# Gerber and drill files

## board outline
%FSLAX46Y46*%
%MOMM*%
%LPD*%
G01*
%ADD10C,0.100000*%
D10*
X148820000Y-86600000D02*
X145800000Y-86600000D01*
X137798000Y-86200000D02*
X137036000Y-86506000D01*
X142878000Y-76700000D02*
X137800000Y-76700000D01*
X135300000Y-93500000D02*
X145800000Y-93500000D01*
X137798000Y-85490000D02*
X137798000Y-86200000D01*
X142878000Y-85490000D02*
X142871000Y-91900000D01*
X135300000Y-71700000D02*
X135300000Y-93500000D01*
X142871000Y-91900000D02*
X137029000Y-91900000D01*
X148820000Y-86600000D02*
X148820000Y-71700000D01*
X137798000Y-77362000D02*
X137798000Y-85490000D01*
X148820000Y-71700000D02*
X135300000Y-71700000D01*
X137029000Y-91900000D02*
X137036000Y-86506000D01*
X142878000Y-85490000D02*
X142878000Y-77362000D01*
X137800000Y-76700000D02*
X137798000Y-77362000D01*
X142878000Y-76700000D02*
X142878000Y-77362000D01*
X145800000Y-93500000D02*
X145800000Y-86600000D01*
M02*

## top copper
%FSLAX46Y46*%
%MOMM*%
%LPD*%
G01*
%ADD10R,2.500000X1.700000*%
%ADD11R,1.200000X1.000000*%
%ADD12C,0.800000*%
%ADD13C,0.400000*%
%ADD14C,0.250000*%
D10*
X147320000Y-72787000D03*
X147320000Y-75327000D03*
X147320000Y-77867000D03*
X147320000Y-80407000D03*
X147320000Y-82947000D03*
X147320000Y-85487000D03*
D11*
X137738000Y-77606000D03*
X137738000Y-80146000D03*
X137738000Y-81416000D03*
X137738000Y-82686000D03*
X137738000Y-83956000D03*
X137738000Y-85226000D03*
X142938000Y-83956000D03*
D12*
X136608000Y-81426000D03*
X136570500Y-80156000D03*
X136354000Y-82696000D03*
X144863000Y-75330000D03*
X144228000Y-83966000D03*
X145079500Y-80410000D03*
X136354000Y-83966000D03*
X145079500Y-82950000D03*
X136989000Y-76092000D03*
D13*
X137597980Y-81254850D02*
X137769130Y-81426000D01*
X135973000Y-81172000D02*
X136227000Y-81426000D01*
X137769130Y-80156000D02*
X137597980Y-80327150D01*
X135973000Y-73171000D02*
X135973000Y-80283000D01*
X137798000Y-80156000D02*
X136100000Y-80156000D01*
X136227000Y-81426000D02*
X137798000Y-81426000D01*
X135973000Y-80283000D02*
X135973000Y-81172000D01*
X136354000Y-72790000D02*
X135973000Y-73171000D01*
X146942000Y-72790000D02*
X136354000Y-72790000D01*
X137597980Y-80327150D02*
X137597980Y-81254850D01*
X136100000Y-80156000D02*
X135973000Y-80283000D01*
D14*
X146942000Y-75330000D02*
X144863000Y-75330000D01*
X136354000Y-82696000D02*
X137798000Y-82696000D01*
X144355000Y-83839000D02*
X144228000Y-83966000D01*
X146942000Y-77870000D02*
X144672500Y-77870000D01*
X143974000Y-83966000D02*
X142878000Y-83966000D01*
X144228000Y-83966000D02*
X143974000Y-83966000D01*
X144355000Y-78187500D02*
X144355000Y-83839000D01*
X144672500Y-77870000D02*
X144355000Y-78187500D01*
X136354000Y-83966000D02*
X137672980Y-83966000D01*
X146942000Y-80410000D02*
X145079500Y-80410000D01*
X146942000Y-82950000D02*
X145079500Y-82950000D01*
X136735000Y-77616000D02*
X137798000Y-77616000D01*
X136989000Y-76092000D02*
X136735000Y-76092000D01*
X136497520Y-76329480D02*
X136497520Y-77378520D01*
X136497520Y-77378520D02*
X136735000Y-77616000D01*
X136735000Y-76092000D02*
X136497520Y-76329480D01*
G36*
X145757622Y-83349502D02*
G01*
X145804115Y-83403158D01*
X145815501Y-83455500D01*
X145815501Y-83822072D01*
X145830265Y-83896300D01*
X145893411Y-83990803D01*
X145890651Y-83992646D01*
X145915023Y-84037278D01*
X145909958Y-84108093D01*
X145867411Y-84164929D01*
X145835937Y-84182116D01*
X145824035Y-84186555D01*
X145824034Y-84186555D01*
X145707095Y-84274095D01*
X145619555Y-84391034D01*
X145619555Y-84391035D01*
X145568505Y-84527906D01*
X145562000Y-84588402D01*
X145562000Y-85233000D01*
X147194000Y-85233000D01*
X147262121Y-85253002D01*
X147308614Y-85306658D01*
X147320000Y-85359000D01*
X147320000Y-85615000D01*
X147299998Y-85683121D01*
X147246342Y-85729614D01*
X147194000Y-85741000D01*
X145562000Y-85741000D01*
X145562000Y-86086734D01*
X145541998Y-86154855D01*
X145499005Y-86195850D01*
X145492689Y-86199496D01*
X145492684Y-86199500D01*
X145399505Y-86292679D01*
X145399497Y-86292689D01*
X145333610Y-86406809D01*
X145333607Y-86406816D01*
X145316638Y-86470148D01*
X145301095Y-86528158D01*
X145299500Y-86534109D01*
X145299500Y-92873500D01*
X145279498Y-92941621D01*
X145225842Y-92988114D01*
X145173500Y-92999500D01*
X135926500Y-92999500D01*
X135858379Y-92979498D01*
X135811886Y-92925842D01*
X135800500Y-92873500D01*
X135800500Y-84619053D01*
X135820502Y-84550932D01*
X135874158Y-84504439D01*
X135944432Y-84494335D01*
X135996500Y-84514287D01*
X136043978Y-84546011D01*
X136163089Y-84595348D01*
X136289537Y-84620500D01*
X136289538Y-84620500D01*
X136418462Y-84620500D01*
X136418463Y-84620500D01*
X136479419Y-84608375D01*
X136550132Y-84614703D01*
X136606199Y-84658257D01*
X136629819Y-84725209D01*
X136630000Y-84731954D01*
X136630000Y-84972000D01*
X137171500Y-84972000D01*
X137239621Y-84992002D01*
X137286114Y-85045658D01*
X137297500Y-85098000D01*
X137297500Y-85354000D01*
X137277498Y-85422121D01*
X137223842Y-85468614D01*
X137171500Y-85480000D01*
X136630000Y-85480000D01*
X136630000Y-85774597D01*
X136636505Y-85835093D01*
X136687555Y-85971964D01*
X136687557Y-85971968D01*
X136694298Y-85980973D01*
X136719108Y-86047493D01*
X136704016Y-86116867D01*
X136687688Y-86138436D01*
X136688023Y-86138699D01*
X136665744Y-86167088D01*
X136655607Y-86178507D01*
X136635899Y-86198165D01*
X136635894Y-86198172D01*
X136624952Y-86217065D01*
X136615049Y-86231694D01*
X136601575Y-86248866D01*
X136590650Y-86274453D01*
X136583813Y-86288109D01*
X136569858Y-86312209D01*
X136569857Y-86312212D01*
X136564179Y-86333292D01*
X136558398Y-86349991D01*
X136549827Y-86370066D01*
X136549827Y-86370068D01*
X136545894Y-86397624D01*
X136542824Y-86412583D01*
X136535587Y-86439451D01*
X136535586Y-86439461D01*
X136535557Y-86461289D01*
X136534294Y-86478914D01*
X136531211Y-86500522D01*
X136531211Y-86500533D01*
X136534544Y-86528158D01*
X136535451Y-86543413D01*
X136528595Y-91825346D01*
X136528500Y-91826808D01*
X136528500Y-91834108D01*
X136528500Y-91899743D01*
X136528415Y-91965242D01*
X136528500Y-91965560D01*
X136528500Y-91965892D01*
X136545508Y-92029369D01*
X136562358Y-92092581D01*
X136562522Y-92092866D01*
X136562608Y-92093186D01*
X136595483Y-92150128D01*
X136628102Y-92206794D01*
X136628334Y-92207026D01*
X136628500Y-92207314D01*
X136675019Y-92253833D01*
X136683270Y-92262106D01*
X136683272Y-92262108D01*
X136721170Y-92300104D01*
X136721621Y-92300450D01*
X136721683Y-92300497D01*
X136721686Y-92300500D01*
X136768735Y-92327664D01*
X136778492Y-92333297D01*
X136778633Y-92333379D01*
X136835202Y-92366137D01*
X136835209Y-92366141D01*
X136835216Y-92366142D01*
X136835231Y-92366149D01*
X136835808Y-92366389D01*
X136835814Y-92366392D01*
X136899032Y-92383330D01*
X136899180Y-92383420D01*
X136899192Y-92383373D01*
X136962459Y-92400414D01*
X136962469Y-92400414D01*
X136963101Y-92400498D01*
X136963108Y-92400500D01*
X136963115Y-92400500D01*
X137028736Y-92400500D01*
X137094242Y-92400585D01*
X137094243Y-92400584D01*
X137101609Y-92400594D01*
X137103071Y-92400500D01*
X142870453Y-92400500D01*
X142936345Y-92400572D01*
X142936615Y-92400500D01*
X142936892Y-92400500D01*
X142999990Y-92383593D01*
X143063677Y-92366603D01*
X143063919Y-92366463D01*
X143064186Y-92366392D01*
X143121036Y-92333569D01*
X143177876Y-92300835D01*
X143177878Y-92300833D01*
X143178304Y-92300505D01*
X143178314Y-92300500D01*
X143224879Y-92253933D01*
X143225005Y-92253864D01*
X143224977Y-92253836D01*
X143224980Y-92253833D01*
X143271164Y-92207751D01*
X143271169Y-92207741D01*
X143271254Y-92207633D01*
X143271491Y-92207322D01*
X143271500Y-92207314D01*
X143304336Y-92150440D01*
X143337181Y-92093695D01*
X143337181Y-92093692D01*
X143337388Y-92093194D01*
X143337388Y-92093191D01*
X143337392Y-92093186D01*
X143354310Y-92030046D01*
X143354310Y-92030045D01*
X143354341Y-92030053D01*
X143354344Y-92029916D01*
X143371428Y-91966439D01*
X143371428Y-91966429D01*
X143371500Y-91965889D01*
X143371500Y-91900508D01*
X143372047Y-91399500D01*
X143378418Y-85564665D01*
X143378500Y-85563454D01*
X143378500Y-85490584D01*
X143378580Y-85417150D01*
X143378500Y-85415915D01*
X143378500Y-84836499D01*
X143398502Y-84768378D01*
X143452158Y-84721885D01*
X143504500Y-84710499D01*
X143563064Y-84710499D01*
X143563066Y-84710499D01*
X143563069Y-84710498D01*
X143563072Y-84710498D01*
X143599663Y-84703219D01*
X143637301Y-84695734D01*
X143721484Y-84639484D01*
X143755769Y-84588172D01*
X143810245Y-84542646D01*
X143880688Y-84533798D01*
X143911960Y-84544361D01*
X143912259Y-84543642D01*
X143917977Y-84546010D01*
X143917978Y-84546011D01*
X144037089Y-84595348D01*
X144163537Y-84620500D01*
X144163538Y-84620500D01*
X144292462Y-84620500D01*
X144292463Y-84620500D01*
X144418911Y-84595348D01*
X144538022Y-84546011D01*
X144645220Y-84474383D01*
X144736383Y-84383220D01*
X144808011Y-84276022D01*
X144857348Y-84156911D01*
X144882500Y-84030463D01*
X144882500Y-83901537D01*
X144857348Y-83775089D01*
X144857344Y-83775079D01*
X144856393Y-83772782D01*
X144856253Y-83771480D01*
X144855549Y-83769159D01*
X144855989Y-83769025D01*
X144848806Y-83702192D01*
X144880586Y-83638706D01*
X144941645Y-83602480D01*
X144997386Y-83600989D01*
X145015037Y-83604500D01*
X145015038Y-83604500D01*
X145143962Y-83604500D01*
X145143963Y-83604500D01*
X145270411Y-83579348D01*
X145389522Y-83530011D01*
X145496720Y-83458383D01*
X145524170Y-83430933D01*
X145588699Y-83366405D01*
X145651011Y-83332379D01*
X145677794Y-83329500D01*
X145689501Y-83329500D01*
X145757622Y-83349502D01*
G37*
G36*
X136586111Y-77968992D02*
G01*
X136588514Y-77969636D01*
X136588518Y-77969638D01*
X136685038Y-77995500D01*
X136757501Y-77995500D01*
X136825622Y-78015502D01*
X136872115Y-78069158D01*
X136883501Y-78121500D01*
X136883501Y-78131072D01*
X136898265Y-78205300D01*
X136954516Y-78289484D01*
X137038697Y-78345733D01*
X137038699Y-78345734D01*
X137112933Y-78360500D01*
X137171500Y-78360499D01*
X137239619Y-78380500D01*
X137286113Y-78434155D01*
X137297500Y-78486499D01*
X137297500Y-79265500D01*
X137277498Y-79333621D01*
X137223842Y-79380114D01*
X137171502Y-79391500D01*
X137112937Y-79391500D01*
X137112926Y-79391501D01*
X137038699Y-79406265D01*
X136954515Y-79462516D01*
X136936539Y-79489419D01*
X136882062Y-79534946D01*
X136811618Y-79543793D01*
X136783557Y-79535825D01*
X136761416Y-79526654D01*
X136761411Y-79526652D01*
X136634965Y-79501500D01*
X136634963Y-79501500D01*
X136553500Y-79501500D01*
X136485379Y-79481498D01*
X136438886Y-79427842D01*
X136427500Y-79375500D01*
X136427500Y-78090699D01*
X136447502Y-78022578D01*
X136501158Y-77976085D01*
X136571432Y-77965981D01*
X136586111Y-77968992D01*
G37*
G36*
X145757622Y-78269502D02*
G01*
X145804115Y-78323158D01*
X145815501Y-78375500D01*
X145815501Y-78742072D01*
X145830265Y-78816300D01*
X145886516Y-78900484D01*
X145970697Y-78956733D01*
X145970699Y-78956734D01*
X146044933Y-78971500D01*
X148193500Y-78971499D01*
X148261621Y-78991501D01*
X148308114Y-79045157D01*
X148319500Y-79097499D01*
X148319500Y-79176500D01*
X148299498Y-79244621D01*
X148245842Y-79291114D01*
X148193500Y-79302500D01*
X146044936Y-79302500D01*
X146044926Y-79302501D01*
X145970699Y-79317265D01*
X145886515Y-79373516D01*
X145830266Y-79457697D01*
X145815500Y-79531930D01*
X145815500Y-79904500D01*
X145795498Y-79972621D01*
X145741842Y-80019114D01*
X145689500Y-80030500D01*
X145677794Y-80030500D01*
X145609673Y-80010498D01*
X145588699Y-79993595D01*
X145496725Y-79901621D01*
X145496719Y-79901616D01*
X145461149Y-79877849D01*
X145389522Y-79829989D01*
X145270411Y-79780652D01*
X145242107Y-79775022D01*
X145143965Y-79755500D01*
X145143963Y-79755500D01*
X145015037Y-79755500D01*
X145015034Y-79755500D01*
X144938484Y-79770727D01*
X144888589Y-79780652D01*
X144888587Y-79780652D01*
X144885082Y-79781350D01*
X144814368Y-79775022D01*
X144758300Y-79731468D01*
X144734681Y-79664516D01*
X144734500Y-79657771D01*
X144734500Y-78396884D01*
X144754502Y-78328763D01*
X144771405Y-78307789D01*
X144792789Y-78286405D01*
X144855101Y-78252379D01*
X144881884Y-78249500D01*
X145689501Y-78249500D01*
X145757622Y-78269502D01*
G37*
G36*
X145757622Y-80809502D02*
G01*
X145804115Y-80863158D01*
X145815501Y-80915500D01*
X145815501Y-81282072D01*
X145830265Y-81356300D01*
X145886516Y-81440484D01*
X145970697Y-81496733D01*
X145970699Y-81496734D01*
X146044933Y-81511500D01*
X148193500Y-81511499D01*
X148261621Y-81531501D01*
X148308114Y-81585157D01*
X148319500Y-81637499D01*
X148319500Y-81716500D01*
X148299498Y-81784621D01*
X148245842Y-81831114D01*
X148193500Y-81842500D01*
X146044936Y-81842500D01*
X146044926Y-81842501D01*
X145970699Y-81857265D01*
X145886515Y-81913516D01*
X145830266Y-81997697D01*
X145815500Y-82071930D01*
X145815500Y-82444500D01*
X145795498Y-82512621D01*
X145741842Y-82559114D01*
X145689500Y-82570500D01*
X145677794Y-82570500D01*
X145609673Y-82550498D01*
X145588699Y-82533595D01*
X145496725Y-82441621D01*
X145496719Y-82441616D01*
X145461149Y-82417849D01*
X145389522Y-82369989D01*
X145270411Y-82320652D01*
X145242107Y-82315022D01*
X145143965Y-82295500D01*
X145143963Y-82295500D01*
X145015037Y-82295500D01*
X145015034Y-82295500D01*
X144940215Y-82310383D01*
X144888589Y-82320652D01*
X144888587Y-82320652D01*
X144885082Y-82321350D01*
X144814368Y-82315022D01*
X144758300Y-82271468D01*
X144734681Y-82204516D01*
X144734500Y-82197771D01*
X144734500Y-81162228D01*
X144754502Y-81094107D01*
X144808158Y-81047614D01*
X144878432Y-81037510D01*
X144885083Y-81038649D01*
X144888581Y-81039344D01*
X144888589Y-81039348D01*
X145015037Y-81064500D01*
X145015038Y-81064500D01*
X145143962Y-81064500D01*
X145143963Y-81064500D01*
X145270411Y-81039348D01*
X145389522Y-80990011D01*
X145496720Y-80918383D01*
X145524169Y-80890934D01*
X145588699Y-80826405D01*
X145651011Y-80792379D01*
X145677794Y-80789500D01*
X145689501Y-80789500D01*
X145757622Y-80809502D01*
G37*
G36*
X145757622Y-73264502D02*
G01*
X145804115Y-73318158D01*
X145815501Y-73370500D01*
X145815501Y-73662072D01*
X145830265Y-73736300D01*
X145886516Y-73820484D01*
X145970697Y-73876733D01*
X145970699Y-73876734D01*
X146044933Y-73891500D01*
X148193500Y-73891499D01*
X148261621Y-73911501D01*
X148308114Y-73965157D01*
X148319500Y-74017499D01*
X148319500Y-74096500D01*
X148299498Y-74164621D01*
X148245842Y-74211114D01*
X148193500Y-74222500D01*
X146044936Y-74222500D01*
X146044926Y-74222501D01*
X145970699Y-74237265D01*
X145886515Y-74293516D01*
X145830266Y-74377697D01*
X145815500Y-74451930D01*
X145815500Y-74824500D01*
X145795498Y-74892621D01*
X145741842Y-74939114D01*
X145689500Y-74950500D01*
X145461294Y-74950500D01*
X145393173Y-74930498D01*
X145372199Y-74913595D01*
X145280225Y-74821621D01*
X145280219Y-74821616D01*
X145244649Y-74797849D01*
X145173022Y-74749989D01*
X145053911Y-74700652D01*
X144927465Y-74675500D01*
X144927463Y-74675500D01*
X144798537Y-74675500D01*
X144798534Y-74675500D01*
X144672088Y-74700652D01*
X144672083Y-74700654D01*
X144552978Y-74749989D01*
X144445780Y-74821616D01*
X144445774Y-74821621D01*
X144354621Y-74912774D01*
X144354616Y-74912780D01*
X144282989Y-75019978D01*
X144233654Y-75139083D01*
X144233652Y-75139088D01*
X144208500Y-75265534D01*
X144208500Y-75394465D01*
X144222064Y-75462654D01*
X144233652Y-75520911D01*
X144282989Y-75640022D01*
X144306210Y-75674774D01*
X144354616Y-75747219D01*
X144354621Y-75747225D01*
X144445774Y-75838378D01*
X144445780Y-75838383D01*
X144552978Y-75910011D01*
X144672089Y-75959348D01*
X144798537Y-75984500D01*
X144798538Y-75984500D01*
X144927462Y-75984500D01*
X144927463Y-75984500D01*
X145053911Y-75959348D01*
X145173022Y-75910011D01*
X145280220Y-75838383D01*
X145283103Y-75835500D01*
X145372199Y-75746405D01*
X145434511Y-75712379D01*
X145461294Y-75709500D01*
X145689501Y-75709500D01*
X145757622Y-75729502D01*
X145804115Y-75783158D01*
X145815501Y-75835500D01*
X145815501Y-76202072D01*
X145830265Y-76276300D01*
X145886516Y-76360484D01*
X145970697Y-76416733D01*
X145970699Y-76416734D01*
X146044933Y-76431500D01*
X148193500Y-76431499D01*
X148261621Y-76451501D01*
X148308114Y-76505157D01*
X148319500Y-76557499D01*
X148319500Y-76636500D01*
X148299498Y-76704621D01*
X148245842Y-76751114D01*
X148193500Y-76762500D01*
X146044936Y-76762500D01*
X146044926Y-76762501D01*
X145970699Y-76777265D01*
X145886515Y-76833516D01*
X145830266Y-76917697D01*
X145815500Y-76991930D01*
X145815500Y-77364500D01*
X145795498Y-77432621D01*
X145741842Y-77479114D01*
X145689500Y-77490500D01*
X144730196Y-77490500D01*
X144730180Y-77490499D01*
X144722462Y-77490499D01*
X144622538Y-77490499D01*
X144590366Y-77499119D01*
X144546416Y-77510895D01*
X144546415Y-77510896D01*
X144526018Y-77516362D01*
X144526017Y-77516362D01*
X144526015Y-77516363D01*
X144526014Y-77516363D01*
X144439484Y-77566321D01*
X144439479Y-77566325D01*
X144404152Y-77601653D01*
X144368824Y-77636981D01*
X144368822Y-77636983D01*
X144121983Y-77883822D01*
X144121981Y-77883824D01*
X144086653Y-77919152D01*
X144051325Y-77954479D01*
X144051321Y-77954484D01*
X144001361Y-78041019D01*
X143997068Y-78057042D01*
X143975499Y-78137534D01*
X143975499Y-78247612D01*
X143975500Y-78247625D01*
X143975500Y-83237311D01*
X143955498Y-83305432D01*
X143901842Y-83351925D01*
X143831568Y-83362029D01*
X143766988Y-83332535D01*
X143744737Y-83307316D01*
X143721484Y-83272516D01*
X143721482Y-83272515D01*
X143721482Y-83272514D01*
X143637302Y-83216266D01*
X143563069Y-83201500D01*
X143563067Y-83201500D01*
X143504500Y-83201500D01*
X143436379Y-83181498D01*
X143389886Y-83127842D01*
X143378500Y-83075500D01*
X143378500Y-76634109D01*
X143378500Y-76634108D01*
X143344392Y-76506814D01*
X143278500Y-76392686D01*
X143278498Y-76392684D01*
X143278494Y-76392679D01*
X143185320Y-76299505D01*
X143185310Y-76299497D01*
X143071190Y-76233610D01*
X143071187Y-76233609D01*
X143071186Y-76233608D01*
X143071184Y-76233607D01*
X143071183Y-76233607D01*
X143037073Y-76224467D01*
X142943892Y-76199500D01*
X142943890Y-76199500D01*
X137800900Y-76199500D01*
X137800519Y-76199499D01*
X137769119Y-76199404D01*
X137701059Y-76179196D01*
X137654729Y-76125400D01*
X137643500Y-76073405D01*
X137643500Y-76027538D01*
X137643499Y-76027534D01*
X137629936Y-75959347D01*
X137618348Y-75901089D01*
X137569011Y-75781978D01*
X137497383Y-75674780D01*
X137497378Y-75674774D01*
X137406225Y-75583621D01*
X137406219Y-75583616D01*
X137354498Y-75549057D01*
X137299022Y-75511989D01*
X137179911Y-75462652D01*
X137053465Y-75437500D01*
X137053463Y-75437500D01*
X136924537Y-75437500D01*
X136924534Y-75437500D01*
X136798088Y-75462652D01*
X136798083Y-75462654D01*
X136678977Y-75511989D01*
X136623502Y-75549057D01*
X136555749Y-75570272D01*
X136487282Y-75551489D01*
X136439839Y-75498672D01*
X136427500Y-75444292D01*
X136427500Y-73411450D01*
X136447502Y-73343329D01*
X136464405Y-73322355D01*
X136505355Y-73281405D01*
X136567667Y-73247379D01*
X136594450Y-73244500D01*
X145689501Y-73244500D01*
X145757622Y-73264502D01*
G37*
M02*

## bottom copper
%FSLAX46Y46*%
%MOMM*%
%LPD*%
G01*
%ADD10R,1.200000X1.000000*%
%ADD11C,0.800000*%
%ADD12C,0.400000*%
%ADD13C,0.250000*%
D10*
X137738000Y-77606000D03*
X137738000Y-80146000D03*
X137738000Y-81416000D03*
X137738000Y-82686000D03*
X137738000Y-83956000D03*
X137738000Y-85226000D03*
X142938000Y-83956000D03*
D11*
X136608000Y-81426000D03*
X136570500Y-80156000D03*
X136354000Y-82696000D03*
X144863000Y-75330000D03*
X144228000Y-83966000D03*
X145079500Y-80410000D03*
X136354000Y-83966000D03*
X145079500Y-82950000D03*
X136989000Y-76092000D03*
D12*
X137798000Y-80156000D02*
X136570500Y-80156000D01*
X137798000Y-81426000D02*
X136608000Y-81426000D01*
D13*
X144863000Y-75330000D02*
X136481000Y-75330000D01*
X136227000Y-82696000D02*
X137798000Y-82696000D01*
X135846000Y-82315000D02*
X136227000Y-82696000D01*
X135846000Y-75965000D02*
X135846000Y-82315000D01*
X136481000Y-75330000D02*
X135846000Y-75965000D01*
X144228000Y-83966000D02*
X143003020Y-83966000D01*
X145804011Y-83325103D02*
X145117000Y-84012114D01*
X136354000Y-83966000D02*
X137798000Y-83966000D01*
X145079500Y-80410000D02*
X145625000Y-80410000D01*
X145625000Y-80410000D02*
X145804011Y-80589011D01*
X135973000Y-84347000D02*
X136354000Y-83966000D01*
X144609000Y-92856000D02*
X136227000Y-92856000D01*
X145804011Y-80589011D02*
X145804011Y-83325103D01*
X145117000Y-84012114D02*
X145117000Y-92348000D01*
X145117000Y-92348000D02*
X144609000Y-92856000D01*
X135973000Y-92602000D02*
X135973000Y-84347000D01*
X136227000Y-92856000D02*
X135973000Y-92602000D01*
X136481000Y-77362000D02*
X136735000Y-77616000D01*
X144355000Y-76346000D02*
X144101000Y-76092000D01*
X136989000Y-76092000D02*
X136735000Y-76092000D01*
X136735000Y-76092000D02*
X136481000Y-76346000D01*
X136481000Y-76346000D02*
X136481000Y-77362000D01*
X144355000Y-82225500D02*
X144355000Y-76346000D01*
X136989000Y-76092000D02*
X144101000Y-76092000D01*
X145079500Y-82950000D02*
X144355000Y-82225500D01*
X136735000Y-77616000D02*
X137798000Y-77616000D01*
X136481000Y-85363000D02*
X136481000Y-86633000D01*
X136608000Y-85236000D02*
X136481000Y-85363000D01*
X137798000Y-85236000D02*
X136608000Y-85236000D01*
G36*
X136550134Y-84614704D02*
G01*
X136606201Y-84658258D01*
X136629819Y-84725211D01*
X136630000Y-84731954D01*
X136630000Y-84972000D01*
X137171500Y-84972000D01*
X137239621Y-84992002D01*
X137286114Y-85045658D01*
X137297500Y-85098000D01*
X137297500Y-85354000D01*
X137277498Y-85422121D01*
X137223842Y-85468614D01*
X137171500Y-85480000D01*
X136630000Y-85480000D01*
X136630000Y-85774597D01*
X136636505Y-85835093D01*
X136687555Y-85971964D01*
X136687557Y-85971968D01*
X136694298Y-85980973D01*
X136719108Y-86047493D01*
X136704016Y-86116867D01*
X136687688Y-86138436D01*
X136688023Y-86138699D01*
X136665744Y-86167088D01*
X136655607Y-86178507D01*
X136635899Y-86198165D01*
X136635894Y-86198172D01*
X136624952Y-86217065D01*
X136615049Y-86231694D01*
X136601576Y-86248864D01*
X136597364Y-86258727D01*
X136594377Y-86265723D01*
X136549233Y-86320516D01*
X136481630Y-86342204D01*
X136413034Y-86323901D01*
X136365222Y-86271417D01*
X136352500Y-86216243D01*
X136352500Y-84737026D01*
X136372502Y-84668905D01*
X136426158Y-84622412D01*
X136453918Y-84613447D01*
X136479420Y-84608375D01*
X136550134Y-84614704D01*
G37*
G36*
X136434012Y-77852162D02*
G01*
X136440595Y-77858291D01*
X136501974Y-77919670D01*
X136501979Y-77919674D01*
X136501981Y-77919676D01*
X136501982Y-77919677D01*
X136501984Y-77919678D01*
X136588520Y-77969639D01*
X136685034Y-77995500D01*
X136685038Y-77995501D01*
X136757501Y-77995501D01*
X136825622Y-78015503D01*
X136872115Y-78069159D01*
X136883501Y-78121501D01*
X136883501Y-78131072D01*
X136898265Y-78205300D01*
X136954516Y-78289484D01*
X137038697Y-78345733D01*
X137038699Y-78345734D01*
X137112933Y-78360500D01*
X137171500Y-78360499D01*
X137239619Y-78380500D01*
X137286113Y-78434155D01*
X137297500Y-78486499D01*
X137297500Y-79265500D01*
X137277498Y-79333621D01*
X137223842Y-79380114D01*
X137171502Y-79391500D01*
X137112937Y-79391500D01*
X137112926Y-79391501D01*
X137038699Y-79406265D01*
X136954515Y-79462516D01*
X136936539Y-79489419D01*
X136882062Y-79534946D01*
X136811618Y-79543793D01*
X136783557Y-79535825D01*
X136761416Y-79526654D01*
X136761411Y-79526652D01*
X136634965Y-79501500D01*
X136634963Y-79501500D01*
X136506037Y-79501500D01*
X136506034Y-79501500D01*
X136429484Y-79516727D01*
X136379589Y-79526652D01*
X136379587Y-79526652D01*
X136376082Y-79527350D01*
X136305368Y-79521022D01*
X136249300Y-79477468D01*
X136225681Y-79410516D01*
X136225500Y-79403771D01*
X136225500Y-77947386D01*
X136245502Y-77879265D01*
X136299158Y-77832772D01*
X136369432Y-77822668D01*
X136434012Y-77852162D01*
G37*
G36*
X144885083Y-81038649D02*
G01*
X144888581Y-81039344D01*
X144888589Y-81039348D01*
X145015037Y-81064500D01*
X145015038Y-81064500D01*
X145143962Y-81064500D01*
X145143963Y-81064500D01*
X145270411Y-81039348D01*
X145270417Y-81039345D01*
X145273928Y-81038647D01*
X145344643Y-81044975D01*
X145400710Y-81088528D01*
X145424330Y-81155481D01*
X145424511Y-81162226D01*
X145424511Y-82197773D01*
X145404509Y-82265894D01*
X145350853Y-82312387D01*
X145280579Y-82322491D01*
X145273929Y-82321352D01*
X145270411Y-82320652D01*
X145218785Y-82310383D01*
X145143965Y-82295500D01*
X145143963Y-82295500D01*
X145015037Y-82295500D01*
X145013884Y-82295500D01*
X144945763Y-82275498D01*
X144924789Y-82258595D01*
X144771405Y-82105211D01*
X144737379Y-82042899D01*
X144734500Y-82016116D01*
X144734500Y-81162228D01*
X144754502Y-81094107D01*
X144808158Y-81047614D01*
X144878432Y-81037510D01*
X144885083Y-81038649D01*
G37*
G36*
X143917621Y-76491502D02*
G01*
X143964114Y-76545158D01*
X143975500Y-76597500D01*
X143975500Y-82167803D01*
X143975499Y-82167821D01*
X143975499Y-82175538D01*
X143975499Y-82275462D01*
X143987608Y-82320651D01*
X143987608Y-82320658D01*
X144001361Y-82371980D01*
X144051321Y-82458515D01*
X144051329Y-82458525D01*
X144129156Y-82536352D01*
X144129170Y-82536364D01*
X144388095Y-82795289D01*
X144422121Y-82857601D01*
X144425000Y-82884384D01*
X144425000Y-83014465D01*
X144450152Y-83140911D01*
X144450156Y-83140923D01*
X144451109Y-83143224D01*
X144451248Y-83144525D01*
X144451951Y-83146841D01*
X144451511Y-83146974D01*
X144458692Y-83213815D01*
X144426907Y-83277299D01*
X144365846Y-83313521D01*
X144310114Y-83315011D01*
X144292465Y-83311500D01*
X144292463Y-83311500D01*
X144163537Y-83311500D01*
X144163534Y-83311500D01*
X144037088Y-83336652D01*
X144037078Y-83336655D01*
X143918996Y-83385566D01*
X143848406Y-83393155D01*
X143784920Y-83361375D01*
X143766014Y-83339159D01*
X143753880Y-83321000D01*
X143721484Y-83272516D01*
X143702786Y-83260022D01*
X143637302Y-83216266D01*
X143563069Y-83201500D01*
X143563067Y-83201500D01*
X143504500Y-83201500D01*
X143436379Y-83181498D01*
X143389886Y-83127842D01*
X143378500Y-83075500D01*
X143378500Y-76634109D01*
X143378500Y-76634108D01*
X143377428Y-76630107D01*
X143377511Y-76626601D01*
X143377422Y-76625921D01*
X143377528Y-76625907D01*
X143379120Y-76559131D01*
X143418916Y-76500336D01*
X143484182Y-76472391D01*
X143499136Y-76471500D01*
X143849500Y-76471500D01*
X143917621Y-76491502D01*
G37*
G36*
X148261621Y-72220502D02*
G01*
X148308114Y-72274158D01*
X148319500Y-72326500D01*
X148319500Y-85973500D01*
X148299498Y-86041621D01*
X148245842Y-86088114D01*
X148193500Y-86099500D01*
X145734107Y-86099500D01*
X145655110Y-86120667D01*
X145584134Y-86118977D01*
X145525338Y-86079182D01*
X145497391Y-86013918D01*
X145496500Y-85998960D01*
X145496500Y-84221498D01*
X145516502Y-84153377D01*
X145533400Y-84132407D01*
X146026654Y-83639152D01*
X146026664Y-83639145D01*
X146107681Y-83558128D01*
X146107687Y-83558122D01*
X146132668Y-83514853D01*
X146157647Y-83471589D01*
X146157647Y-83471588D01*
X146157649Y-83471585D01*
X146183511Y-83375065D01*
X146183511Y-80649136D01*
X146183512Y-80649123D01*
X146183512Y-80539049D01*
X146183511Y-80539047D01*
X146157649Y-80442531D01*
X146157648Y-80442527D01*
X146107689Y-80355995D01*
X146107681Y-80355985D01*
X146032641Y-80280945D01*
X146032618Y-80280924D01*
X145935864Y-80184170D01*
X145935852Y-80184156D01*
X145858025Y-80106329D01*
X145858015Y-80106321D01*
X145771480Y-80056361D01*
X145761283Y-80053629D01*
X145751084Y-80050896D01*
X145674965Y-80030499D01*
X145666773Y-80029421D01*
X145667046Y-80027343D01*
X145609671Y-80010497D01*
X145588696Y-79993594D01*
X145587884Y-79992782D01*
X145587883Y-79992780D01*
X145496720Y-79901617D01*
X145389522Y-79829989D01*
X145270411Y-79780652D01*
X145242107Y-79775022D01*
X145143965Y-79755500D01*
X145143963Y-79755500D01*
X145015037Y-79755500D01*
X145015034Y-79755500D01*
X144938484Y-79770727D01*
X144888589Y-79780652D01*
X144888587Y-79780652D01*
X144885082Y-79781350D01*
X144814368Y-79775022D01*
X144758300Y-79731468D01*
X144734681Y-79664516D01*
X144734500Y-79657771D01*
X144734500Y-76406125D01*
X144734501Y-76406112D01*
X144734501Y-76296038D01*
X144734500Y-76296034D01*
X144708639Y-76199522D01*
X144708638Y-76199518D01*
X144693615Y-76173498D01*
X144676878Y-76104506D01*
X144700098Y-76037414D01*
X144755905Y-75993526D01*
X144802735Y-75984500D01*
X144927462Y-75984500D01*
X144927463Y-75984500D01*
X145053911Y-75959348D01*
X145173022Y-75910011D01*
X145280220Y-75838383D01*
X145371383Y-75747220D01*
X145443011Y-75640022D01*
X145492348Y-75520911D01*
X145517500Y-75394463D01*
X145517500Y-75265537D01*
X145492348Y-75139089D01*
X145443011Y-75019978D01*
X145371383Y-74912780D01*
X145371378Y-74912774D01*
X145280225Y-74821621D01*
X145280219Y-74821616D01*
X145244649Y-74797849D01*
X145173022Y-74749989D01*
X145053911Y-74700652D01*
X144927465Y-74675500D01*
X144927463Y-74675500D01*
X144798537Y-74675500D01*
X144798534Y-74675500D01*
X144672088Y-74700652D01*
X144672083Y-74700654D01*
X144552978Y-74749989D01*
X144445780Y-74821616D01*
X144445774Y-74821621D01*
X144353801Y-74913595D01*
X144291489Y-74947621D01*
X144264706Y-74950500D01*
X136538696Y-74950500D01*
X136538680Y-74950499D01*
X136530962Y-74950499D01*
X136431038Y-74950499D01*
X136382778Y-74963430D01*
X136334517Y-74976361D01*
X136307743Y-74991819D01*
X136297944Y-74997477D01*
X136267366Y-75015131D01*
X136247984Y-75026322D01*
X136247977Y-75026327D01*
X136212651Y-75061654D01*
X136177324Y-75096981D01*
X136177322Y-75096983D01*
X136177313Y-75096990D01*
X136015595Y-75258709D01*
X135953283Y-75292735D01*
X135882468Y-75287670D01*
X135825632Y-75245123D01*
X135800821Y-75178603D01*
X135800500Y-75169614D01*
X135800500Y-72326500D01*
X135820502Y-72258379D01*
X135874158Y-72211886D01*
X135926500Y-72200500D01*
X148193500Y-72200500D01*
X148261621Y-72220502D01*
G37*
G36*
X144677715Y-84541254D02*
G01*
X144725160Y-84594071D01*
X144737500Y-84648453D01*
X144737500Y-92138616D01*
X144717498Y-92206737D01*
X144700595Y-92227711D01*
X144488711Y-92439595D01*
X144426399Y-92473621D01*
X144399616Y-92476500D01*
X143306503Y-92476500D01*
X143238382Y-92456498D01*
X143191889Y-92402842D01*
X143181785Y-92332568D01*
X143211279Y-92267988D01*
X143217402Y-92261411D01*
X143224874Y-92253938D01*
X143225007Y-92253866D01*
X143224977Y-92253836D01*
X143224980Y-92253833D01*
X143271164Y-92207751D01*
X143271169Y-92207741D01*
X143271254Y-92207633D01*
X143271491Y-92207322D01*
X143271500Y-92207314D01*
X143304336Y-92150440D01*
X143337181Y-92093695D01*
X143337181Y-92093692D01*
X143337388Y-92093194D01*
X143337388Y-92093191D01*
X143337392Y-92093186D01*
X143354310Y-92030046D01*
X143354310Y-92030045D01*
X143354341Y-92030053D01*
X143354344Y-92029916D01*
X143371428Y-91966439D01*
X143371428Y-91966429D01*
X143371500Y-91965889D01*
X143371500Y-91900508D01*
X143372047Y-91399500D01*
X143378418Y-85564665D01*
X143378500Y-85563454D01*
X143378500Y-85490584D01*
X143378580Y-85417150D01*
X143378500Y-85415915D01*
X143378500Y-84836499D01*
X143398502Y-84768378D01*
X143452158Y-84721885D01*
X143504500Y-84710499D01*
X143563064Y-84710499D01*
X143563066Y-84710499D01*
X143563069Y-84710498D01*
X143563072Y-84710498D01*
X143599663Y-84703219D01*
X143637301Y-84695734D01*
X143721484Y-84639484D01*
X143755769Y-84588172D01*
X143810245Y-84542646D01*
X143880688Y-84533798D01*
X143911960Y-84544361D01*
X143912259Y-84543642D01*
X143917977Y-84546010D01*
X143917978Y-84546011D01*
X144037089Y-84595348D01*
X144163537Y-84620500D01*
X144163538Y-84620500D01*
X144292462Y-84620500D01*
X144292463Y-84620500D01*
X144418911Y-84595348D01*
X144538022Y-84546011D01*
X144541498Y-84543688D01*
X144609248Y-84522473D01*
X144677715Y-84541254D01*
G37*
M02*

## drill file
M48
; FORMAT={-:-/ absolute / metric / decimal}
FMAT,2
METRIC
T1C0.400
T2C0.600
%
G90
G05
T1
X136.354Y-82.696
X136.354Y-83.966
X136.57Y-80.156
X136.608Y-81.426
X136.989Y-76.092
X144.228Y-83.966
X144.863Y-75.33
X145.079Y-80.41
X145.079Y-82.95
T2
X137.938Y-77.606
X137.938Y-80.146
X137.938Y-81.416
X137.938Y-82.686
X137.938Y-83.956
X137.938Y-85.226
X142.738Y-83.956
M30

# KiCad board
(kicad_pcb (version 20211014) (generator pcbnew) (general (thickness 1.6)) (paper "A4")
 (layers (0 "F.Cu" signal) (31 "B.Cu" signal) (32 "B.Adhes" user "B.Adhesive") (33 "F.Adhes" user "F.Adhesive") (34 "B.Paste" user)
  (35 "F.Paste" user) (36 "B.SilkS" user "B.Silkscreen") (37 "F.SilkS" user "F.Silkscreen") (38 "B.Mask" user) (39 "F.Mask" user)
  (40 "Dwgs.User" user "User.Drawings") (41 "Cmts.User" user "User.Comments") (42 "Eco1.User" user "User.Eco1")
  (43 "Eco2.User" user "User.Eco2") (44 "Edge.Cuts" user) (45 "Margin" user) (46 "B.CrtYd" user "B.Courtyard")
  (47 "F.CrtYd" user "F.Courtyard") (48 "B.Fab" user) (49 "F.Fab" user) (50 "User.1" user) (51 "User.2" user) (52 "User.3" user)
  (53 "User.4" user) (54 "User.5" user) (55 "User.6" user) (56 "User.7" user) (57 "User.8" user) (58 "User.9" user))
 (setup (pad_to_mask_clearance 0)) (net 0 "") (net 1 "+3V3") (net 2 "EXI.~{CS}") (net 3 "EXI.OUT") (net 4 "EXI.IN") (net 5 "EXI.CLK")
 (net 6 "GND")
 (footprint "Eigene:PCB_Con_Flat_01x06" (layer "F.Cu") (at 147.32 79.137)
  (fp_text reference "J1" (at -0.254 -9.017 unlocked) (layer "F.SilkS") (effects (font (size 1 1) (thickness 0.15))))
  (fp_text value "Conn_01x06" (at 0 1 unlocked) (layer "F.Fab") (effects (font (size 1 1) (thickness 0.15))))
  (pad "1" smd rect (at 0 -6.35) (size 2.5 1.7) (layers "F.Cu" "F.Paste" "F.Mask") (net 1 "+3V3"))
  (pad "2" smd rect (at 0 -3.81) (size 2.5 1.7) (layers "F.Cu" "F.Paste" "F.Mask") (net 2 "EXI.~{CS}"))
  (pad "3" smd rect (at 0 -1.27) (size 2.5 1.7) (layers "F.Cu" "F.Paste" "F.Mask") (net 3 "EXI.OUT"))
  (pad "4" smd rect (at 0 1.27) (size 2.5 1.7) (layers "F.Cu" "F.Paste" "F.Mask") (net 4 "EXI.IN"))
  (pad "5" smd rect (at 0 3.81) (size 2.5 1.7) (layers "F.Cu" "F.Paste" "F.Mask") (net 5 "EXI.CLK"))
  (pad "6" smd rect (at 0 6.35) (size 2.5 1.7) (layers "F.Cu" "F.Paste" "F.Mask") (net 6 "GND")))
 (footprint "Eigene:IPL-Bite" (layer "F.Cu") (at 140.338 81.426)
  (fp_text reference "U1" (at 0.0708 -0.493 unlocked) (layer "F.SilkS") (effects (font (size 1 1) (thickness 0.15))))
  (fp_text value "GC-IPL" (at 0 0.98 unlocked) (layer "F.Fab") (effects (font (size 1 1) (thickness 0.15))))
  (pad "1" thru_hole rect (at -2.4 -3.82) (size 1.2 1) (drill 0.6 (offset -0.2 0)) (layers *.Cu *.Mask) (remove_unused_layers)
   (keep_end_layers) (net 5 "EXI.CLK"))
  (pad "3" thru_hole rect (at -2.4 -1.28) (size 1.2 1) (drill 0.6 (offset -0.2 0)) (layers *.Cu *.Mask) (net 1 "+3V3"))
  (pad "4" thru_hole rect (at -2.4 -0.01) (size 1.2 1) (drill 0.6 (offset -0.2 0)) (layers *.Cu *.Mask) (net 1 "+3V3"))
  (pad "5" thru_hole rect (at -2.4 1.26) (size 1.2 1) (drill 0.6 (offset -0.2 0)) (layers *.Cu *.Mask) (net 2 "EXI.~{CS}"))
  (pad "6" thru_hole rect (at -2.4 2.53) (size 1.2 1) (drill 0.6 (offset -0.2 0)) (layers *.Cu *.Mask) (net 4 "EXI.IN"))
  (pad "7" thru_hole rect (at -2.4 3.8) (size 1.2 1) (drill 0.6 (offset -0.2 0)) (layers *.Cu *.Mask) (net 6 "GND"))
  (pad "9" thru_hole rect (at 2.4 2.53 180) (size 1.2 1) (drill 0.6 (offset -0.2 0)) (layers *.Cu *.Mask) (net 3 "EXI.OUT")))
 (gr_line (start 148.82 86.6) (end 145.8 86.6) (layer "Edge.Cuts") (width 0.1))
 (gr_line (start 137.798 86.2) (end 137.036 86.506) (layer "Edge.Cuts") (width 0.1))
 (gr_line (start 142.878 76.7) (end 137.8 76.7) (layer "Edge.Cuts") (width 0.1))
 (gr_line (start 135.3 93.5) (end 145.8 93.5) (layer "Edge.Cuts") (width 0.1))
 (gr_line (start 137.798 85.49) (end 137.798 86.2) (layer "Edge.Cuts") (width 0.1))
 (gr_line (start 142.878 85.49) (end 142.871 91.9) (layer "Edge.Cuts") (width 0.1))
 (gr_line (start 135.3 71.7) (end 135.3 93.5) (layer "Edge.Cuts") (width 0.1))
 (gr_line (start 142.871 91.9) (end 137.029 91.9) (layer "Edge.Cuts") (width 0.1))
 (gr_line (start 148.82 86.6) (end 148.82 71.7) (layer "Edge.Cuts") (width 0.1))
 (gr_line (start 137.798 77.362) (end 137.798 85.49) (layer "Edge.Cuts") (width 0.1))
 (gr_line (start 148.82 71.7) (end 135.3 71.7) (layer "Edge.Cuts") (width 0.1))
 (gr_line (start 137.029 91.9) (end 137.036 86.506) (layer "Edge.Cuts") (width 0.1))
 (gr_line (start 142.878 85.49) (end 142.878 77.362) (layer "Edge.Cuts") (width 0.1))
 (gr_line (start 137.8 76.7) (end 137.798 77.362) (layer "Edge.Cuts") (width 0.1))
 (gr_line (start 142.878 76.7) (end 142.878 77.362) (layer "Edge.Cuts") (width 0.1))
 (gr_line (start 145.8 93.5) (end 145.8 86.6) (layer "Edge.Cuts") (width 0.1))
 (segment (start 137.59798 81.25485) (end 137.76913 81.426) (width 0.4) (layer "F.Cu") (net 1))
 (segment (start 135.973 81.172) (end 136.227 81.426) (width 0.4) (layer "F.Cu") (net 1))
 (segment (start 137.76913 80.156) (end 137.59798 80.32715) (width 0.4) (layer "F.Cu") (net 1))
 (segment (start 135.973 73.171) (end 135.973 80.283) (width 0.4) (layer "F.Cu") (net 1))
 (segment (start 137.798 80.156) (end 136.1 80.156) (width 0.4) (layer "F.Cu") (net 1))
 (segment (start 136.227 81.426) (end 137.798 81.426) (width 0.4) (layer "F.Cu") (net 1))
 (segment (start 135.973 80.283) (end 135.973 81.172) (width 0.4) (layer "F.Cu") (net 1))
 (segment (start 136.354 72.79) (end 135.973 73.171) (width 0.4) (layer "F.Cu") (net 1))
 (segment (start 146.942 72.79) (end 136.354 72.79) (width 0.4) (layer "F.Cu") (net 1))
 (segment (start 137.59798 80.32715) (end 137.59798 81.25485) (width 0.4) (layer "F.Cu") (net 1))
 (segment (start 136.1 80.156) (end 135.973 80.283) (width 0.4) (layer "F.Cu") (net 1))
 (via (at 136.608 81.426) (size 0.8) (drill 0.4) (layers "F.Cu" "B.Cu") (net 1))
 (via (at 136.5705 80.156) (size 0.8) (drill 0.4) (layers "F.Cu" "B.Cu") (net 1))
 (segment (start 137.798 80.156) (end 136.5705 80.156) (width 0.4) (layer "B.Cu") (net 1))
 (segment (start 137.798 81.426) (end 136.608 81.426) (width 0.4) (layer "B.Cu") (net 1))
 (segment (start 146.942 75.33) (end 144.863 75.33) (width 0.25) (layer "F.Cu") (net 2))
 (segment (start 136.354 82.696) (end 137.798 82.696) (width 0.25) (layer "F.Cu") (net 2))
 (via (at 136.354 82.696) (size 0.8) (drill 0.4) (layers "F.Cu" "B.Cu") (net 2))
 (via (at 144.863 75.33) (size 0.8) (drill 0.4) (layers "F.Cu" "B.Cu") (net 2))
 (segment (start 144.863 75.33) (end 136.481 75.33) (width 0.25) (layer "B.Cu") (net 2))
 (segment (start 136.227 82.696) (end 137.798 82.696) (width 0.25) (layer "B.Cu") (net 2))
 (segment (start 135.846 82.315) (end 136.227 82.696) (width 0.25) (layer "B.Cu") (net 2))
 (segment (start 135.846 75.965) (end 135.846 82.315) (width 0.25) (layer "B.Cu") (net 2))
 (segment (start 136.481 75.33) (end 135.846 75.965) (width 0.25) (layer "B.Cu") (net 2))
 (segment (start 144.355 83.839) (end 144.228 83.966) (width 0.25) (layer "F.Cu") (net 3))
 (segment (start 146.942 77.87) (end 144.6725 77.87) (width 0.25) (layer "F.Cu") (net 3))
 (segment (start 143.974 83.966) (end 142.878 83.966) (width 0.25) (layer "F.Cu") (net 3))
 (segment (start 144.228 83.966) (end 143.974 83.966) (width 0.25) (layer "F.Cu") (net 3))
 (segment (start 144.355 78.1875) (end 144.355 83.839) (width 0.25) (layer "F.Cu") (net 3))
 (segment (start 144.6725 77.87) (end 144.355 78.1875) (width 0.25) (layer "F.Cu") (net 3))
 (via (at 144.228 83.966) (size 0.8) (drill 0.4) (layers "F.Cu" "B.Cu") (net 3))
 (segment (start 144.228 83.966) (end 143.00302 83.966) (width 0.25) (layer "B.Cu") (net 3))
 (segment (start 136.354 83.966) (end 137.67298 83.966) (width 0.25) (layer "F.Cu") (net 4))
 (segment (start 146.942 80.41) (end 145.0795 80.41) (width 0.25) (layer "F.Cu") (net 4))
 (via (at 145.0795 80.41) (size 0.8) (drill 0.4) (layers "F.Cu" "B.Cu") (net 4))
 (via (at 136.354 83.966) (size 0.8) (drill 0.4) (layers "F.Cu" "B.Cu") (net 4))
 (segment (start 145.804011 83.325103) (end 145.117 84.012114) (width 0.25) (layer "B.Cu") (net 4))
 (segment (start 136.354 83.966) (end 137.798 83.966) (width 0.25) (layer "B.Cu") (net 4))
 (segment (start 145.0795 80.41) (end 145.625 80.41) (width 0.25) (layer "B.Cu") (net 4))
 (segment (start 145.625 80.41) (end 145.804011 80.589011) (width 0.25) (layer "B.Cu") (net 4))
 (segment (start 135.973 84.347) (end 136.354 83.966) (width 0.25) (layer "B.Cu") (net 4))
 (segment (start 144.609 92.856) (end 136.227 92.856) (width 0.25) (layer "B.Cu") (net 4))
 (segment (start 145.804011 80.589011) (end 145.804011 83.325103) (width 0.25) (layer "B.Cu") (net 4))
 (segment (start 145.117 84.012114) (end 145.117 92.348) (width 0.25) (layer "B.Cu") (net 4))
 (segment (start 145.117 92.348) (end 144.609 92.856) (width 0.25) (layer "B.Cu") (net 4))
 (segment (start 135.973 92.602) (end 135.973 84.347) (width 0.25) (layer "B.Cu") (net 4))
 (segment (start 136.227 92.856) (end 135.973 92.602) (width 0.25) (layer "B.Cu") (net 4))
 (segment (start 146.942 82.95) (end 145.0795 82.95) (width 0.25) (layer "F.Cu") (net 5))
 (segment (start 136.735 77.616) (end 137.798 77.616) (width 0.25) (layer "F.Cu") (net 5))
 (segment (start 136.989 76.092) (end 136.735 76.092) (width 0.25) (layer "F.Cu") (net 5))
 (segment (start 136.49752 76.32948) (end 136.49752 77.37852) (width 0.25) (layer "F.Cu") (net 5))
 (segment (start 136.49752 77.37852) (end 136.735 77.616) (width 0.25) (layer "F.Cu") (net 5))
 (segment (start 136.735 76.092) (end 136.49752 76.32948) (width 0.25) (layer "F.Cu") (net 5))
 (via (at 145.0795 82.95) (size 0.8) (drill 0.4) (layers "F.Cu" "B.Cu") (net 5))
 (via (at 136.989 76.092) (size 0.8) (drill 0.4) (layers "F.Cu" "B.Cu") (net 5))
 (segment (start 136.481 77.362) (end 136.735 77.616) (width 0.25) (layer "B.Cu") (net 5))
 (segment (start 144.355 76.346) (end 144.101 76.092) (width 0.25) (layer "B.Cu") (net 5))
 (segment (start 136.989 76.092) (end 136.735 76.092) (width 0.25) (layer "B.Cu") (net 5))
 (segment (start 136.735 76.092) (end 136.481 76.346) (width 0.25) (layer "B.Cu") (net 5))
 (segment (start 136.481 76.346) (end 136.481 77.362) (width 0.25) (layer "B.Cu") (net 5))
 (segment (start 144.355 82.2255) (end 144.355 76.346) (width 0.25) (layer "B.Cu") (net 5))
 (segment (start 136.989 76.092) (end 144.101 76.092) (width 0.25) (layer "B.Cu") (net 5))
 (segment (start 145.0795 82.95) (end 144.355 82.2255) (width 0.25) (layer "B.Cu") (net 5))
 (segment (start 136.735 77.616) (end 137.798 77.616) (width 0.25) (layer "B.Cu") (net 5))
 (segment (start 136.481 85.363) (end 136.481 86.633) (width 0.25) (layer "B.Cu") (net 6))
 (segment (start 136.608 85.236) (end 136.481 85.363) (width 0.25) (layer "B.Cu") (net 6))
 (segment (start 137.798 85.236) (end 136.608 85.236) (width 0.25) (layer "B.Cu") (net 6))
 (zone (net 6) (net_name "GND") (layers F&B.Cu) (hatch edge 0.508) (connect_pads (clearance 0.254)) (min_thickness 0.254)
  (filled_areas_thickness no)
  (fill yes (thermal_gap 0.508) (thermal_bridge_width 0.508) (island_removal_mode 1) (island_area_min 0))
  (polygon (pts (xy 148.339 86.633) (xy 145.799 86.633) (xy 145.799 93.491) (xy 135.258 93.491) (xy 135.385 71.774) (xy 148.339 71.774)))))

